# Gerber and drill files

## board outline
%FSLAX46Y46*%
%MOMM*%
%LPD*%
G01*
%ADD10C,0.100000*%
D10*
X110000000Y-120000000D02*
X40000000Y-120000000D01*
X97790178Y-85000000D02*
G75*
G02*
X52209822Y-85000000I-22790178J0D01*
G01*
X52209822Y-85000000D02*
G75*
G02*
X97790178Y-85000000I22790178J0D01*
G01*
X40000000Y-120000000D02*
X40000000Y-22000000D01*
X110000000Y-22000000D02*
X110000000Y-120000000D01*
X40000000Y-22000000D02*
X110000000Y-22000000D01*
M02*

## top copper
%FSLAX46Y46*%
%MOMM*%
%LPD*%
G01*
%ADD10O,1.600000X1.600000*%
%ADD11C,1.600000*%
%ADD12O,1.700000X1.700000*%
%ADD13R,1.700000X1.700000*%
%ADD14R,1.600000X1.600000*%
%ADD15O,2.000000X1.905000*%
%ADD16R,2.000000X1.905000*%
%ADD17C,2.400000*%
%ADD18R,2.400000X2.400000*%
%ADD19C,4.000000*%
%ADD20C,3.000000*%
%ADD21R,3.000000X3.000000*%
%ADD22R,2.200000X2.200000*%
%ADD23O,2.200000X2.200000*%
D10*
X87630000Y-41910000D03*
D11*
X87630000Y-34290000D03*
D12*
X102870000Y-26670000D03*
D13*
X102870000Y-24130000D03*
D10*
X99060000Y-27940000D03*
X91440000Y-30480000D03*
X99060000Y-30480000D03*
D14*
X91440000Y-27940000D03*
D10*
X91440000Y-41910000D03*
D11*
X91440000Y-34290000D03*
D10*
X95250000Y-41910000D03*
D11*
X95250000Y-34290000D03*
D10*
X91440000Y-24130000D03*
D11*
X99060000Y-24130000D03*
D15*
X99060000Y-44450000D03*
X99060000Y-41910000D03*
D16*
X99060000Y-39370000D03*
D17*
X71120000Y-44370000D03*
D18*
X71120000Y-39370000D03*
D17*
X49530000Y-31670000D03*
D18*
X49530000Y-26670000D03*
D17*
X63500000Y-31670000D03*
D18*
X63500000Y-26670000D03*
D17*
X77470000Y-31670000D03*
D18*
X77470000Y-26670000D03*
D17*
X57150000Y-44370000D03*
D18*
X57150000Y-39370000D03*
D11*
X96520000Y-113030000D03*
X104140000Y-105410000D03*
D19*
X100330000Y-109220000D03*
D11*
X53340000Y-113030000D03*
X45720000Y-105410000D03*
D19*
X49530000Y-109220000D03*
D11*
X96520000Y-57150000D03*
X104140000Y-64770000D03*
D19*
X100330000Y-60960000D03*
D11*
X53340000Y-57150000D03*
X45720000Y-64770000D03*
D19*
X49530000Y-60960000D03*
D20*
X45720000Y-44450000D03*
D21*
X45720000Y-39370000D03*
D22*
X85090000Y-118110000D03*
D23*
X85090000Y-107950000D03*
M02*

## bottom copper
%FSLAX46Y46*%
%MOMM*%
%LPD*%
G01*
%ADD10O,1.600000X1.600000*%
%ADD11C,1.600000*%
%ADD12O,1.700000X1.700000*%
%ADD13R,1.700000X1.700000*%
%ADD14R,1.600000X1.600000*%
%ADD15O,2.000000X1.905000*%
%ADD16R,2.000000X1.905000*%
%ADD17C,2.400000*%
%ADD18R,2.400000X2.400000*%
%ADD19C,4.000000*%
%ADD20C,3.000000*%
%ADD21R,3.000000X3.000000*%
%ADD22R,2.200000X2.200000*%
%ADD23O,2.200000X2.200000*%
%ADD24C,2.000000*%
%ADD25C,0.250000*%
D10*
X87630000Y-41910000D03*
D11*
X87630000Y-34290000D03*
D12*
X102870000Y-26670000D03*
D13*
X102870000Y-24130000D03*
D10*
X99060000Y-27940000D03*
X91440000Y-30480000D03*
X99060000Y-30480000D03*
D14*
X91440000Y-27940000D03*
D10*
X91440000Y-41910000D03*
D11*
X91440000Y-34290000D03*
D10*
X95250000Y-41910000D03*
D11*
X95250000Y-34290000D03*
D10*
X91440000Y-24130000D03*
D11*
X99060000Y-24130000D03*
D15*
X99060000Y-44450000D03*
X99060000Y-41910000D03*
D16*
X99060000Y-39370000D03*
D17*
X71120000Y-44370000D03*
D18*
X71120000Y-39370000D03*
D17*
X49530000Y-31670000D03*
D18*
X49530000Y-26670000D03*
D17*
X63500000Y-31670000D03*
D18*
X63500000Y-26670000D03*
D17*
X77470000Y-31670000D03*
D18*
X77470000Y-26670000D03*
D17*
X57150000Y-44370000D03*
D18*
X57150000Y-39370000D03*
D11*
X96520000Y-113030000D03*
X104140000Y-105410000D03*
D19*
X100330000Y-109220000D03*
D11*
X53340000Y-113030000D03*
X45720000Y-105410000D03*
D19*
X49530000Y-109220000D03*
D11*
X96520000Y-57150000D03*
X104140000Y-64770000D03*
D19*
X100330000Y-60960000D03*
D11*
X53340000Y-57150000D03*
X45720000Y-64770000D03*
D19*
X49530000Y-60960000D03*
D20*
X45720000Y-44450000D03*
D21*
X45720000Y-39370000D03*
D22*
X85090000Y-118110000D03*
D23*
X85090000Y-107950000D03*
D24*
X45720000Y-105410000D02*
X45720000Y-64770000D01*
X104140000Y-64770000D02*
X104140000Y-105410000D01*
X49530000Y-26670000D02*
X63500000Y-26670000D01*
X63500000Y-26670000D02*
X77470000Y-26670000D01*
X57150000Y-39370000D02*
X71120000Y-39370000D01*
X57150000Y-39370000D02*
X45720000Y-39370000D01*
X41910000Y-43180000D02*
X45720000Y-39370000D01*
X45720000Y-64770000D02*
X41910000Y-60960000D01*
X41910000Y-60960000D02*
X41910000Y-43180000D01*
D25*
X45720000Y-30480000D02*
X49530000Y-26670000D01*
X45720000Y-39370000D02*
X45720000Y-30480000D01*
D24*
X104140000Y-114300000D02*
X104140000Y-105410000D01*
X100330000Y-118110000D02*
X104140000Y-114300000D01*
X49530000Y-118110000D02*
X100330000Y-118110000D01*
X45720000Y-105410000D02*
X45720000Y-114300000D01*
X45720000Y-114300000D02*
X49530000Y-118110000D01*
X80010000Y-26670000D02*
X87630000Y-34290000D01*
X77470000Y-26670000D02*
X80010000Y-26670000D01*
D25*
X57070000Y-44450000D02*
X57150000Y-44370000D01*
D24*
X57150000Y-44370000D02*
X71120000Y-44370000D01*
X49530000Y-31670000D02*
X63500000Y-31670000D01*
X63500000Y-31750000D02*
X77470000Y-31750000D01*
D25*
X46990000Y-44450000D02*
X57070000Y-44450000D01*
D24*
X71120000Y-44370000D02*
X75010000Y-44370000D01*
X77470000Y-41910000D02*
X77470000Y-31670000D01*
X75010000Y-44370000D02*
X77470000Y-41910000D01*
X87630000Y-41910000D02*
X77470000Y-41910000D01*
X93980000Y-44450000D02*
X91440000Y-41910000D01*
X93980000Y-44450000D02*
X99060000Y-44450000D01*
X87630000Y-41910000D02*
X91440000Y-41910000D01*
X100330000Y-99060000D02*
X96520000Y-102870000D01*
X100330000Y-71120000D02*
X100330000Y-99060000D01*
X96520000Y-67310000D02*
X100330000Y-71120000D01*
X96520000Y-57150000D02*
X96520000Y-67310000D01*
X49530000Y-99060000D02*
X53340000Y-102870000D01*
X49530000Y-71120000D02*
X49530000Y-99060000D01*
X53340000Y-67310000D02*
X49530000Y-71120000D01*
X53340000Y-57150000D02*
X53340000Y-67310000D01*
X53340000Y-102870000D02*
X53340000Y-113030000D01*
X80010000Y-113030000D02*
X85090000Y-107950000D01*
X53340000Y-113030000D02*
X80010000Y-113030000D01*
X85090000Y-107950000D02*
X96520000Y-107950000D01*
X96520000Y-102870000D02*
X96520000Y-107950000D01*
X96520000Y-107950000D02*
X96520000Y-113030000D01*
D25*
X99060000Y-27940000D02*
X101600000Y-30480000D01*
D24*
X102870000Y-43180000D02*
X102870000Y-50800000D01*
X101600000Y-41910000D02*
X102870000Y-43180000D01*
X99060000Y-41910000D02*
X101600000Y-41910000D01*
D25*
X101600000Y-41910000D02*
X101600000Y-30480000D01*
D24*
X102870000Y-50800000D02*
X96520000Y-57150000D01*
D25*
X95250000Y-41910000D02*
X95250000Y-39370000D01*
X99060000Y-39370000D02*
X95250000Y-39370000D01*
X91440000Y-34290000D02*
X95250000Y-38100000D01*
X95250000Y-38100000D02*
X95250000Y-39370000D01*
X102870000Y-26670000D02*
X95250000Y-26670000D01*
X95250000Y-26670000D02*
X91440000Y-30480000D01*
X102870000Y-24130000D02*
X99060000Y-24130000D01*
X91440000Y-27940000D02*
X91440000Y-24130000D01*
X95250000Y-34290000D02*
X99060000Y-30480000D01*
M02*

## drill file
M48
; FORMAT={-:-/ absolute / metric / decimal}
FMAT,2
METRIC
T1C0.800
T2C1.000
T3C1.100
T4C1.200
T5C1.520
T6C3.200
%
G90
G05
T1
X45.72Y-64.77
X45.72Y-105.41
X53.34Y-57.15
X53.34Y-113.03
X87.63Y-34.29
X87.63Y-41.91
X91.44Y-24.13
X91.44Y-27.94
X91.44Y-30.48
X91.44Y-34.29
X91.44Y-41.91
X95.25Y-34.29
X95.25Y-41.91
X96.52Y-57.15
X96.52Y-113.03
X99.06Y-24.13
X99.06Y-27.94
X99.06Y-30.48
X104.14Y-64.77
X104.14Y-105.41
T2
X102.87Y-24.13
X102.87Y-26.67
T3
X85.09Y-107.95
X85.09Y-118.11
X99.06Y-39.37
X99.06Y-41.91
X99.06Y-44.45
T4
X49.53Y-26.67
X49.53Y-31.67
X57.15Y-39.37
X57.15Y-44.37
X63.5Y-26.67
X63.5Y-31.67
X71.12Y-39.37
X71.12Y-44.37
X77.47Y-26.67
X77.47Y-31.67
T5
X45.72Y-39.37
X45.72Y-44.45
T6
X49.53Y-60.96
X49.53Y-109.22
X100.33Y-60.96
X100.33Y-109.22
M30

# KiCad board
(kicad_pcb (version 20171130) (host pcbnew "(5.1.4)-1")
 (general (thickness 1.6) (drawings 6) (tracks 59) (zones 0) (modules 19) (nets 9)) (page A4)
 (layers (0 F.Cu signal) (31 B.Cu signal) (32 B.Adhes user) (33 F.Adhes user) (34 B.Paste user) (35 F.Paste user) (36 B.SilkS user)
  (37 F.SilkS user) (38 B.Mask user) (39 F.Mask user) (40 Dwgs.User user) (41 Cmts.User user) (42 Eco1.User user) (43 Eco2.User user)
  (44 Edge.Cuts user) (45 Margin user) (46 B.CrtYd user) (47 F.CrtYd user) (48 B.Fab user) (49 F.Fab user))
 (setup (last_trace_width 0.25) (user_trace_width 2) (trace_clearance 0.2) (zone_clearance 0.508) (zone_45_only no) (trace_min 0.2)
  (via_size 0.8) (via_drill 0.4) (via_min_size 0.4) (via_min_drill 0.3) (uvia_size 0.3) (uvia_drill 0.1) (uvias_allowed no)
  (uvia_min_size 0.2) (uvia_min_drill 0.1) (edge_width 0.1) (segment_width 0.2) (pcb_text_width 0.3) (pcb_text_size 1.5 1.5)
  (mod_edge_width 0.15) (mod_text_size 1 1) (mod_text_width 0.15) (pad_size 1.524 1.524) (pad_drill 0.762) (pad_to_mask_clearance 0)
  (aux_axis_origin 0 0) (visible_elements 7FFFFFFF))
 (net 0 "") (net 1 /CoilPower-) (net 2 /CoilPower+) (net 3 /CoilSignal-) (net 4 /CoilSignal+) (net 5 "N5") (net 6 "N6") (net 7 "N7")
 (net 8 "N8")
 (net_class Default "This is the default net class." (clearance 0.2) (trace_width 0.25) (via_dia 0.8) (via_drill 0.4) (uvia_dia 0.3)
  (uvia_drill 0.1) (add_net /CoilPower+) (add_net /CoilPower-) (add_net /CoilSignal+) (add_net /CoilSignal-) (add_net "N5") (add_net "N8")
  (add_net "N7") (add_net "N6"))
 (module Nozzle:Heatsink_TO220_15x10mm (layer F.Cu) (at 102.87 41.91 270)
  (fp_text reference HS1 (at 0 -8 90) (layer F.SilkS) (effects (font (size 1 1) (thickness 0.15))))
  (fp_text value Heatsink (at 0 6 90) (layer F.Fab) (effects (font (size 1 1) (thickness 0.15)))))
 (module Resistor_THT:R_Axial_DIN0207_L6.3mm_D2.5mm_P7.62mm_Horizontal (layer F.Cu) (at 87.63 34.29 270)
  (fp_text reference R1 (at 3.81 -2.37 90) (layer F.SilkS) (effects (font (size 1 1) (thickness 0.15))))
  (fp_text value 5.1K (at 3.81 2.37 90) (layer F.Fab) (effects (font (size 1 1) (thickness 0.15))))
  (pad 2 thru_hole oval (at 7.62 0 270) (size 1.6 1.6) (drill 0.8) (layers *.Cu *.Mask) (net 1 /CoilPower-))
  (pad 1 thru_hole circle (at 0 0 270) (size 1.6 1.6) (drill 0.8) (layers *.Cu *.Mask) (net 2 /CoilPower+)))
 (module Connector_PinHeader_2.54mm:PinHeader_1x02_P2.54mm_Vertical (layer F.Cu) (at 102.87 24.13)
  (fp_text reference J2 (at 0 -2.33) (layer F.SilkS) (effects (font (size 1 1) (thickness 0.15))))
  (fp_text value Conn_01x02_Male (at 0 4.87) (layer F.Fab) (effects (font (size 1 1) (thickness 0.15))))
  (pad 2 thru_hole oval (at 0 2.54) (size 1.7 1.7) (drill 1) (layers *.Cu *.Mask) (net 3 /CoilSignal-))
  (pad 1 thru_hole rect (at 0 0) (size 1.7 1.7) (drill 1) (layers *.Cu *.Mask) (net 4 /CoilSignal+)))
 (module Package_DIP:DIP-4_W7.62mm (layer F.Cu) (at 91.44 27.94)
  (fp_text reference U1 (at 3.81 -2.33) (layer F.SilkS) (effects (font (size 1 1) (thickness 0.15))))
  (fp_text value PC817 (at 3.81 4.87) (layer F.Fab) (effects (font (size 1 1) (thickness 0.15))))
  (pad 4 thru_hole oval (at 7.62 0) (size 1.6 1.6) (drill 0.8) (layers *.Cu *.Mask) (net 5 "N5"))
  (pad 2 thru_hole oval (at 0 2.54) (size 1.6 1.6) (drill 0.8) (layers *.Cu *.Mask) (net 3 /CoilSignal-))
  (pad 3 thru_hole oval (at 7.62 2.54) (size 1.6 1.6) (drill 0.8) (layers *.Cu *.Mask) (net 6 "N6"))
  (pad 1 thru_hole rect (at 0 0) (size 1.6 1.6) (drill 0.8) (layers *.Cu *.Mask) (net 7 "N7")))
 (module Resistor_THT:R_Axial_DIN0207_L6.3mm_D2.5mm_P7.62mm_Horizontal (layer F.Cu) (at 91.44 34.29 270)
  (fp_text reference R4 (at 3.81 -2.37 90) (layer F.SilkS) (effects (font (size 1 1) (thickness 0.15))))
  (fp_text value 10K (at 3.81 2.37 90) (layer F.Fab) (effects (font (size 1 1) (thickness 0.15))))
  (pad 2 thru_hole oval (at 7.62 0 270) (size 1.6 1.6) (drill 0.8) (layers *.Cu *.Mask) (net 1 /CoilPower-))
  (pad 1 thru_hole circle (at 0 0 270) (size 1.6 1.6) (drill 0.8) (layers *.Cu *.Mask) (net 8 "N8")))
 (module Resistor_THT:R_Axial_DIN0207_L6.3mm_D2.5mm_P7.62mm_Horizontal (layer F.Cu) (at 95.25 34.29 270)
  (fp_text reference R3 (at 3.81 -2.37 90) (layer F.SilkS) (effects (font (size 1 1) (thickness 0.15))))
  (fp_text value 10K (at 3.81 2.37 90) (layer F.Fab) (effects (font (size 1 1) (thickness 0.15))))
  (pad 2 thru_hole oval (at 7.62 0 270) (size 1.6 1.6) (drill 0.8) (layers *.Cu *.Mask) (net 8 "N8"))
  (pad 1 thru_hole circle (at 0 0 270) (size 1.6 1.6) (drill 0.8) (layers *.Cu *.Mask) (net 6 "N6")))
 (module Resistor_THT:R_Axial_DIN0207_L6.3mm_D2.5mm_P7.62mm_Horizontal (layer F.Cu) (at 99.06 24.13 180)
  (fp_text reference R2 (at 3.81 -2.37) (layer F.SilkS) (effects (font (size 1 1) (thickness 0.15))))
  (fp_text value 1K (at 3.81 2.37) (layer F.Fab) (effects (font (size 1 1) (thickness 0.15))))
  (pad 2 thru_hole oval (at 7.62 0 180) (size 1.6 1.6) (drill 0.8) (layers *.Cu *.Mask) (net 7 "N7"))
  (pad 1 thru_hole circle (at 0 0 180) (size 1.6 1.6) (drill 0.8) (layers *.Cu *.Mask) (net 4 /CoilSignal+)))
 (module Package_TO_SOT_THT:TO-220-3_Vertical (layer F.Cu) (at 99.06 39.37 270)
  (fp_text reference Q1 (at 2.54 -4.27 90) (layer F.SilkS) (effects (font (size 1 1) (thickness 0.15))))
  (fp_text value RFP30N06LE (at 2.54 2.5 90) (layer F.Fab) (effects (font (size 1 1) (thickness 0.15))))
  (pad 3 thru_hole oval (at 5.08 0 270) (size 1.905 2) (drill 1.1) (layers *.Cu *.Mask) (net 1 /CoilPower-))
  (pad 2 thru_hole oval (at 2.54 0 270) (size 1.905 2) (drill 1.1) (layers *.Cu *.Mask) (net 5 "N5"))
  (pad 1 thru_hole rect (at 0 0 270) (size 1.905 2) (drill 1.1) (layers *.Cu *.Mask) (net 8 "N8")))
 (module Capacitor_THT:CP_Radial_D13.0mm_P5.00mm (layer F.Cu) (at 71.12 39.37 270)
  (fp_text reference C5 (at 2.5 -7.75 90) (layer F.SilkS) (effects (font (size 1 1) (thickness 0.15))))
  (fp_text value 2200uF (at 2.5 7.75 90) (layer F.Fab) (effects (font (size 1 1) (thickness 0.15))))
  (pad 2 thru_hole circle (at 5 0 270) (size 2.4 2.4) (drill 1.2) (layers *.Cu *.Mask) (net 1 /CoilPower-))
  (pad 1 thru_hole rect (at 0 0 270) (size 2.4 2.4) (drill 1.2) (layers *.Cu *.Mask) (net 2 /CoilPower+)))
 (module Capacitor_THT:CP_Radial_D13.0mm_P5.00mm (layer F.Cu) (at 49.53 26.67 270)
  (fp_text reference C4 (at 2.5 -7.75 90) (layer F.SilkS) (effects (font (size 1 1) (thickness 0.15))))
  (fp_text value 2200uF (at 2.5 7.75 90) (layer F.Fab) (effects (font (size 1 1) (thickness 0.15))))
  (pad 2 thru_hole circle (at 5 0 270) (size 2.4 2.4) (drill 1.2) (layers *.Cu *.Mask) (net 1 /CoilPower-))
  (pad 1 thru_hole rect (at 0 0 270) (size 2.4 2.4) (drill 1.2) (layers *.Cu *.Mask) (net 2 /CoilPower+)))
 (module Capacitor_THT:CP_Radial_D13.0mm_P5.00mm (layer F.Cu) (at 63.5 26.67 270)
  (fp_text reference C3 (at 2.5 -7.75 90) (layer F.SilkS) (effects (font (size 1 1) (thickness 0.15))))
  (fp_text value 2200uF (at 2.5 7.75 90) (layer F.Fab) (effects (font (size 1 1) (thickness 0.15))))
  (pad 2 thru_hole circle (at 5 0 270) (size 2.4 2.4) (drill 1.2) (layers *.Cu *.Mask) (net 1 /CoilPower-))
  (pad 1 thru_hole rect (at 0 0 270) (size 2.4 2.4) (drill 1.2) (layers *.Cu *.Mask) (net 2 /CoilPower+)))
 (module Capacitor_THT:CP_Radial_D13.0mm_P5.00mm (layer F.Cu) (at 77.47 26.67 270)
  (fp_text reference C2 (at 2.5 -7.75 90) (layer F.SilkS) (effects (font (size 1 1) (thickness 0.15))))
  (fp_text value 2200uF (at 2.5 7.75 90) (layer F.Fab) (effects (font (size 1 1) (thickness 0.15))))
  (pad 2 thru_hole circle (at 5 0 270) (size 2.4 2.4) (drill 1.2) (layers *.Cu *.Mask) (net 1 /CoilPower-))
  (pad 1 thru_hole rect (at 0 0 270) (size 2.4 2.4) (drill 1.2) (layers *.Cu *.Mask) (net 2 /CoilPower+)))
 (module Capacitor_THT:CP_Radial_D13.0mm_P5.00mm (layer F.Cu) (at 57.15 39.37 270)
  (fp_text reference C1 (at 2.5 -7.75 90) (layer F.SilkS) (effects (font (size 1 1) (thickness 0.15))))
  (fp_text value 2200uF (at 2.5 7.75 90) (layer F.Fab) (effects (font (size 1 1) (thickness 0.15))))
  (pad 2 thru_hole circle (at 5 0 270) (size 2.4 2.4) (drill 1.2) (layers *.Cu *.Mask) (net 1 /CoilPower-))
  (pad 1 thru_hole rect (at 0 0 270) (size 2.4 2.4) (drill 1.2) (layers *.Cu *.Mask) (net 2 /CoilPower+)))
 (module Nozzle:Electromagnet (layer F.Cu) (at 100.33 109.22 180)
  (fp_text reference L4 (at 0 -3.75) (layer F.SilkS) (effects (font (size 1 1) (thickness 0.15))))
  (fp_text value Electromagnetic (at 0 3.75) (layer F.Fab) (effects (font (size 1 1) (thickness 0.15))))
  (pad 2 thru_hole circle (at 3.81 -3.81 180) (size 1.6 1.6) (drill 0.8) (layers *.Cu *.Mask) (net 5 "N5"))
  (pad 1 thru_hole circle (at -3.81 3.81 180) (size 1.6 1.6) (drill 0.8) (layers *.Cu *.Mask) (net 2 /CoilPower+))
  (pad 3 thru_hole circle (at 0 0 180) (size 4 4) (drill 3.2) (layers *.Cu *.Mask)))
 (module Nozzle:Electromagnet (layer F.Cu) (at 49.53 109.22 270)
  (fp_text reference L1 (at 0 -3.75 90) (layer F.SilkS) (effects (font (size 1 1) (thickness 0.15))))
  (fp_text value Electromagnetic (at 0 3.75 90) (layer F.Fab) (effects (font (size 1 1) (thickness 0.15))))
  (pad 2 thru_hole circle (at 3.81 -3.81 270) (size 1.6 1.6) (drill 0.8) (layers *.Cu *.Mask) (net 5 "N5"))
  (pad 1 thru_hole circle (at -3.81 3.81 270) (size 1.6 1.6) (drill 0.8) (layers *.Cu *.Mask) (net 2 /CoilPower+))
  (pad 3 thru_hole circle (at 0 0 270) (size 4 4) (drill 3.2) (layers *.Cu *.Mask)))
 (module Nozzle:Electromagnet (layer F.Cu) (at 100.33 60.96 90)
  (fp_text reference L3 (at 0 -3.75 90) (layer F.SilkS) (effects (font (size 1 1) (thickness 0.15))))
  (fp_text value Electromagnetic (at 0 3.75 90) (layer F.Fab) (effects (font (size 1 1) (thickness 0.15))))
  (pad 2 thru_hole circle (at 3.81 -3.81 90) (size 1.6 1.6) (drill 0.8) (layers *.Cu *.Mask) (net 5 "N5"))
  (pad 1 thru_hole circle (at -3.81 3.81 90) (size 1.6 1.6) (drill 0.8) (layers *.Cu *.Mask) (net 2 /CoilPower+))
  (pad 3 thru_hole circle (at 0 0 90) (size 4 4) (drill 3.2) (layers *.Cu *.Mask)))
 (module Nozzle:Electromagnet (layer F.Cu) (at 49.53 60.96)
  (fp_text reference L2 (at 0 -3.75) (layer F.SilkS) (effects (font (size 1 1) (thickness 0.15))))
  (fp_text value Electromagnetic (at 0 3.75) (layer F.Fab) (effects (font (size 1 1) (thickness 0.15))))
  (pad 2 thru_hole circle (at 3.81 -3.81) (size 1.6 1.6) (drill 0.8) (layers *.Cu *.Mask) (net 5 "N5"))
  (pad 1 thru_hole circle (at -3.81 3.81) (size 1.6 1.6) (drill 0.8) (layers *.Cu *.Mask) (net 2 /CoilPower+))
  (pad 3 thru_hole circle (at 0 0) (size 4 4) (drill 3.2) (layers *.Cu *.Mask)))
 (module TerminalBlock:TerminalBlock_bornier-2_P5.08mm (layer F.Cu) (at 45.72 39.37 270)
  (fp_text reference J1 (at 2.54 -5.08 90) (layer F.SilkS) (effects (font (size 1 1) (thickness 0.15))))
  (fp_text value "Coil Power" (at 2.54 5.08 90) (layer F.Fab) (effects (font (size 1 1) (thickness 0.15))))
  (pad 2 thru_hole circle (at 5.08 0 270) (size 3 3) (drill 1.52) (layers *.Cu *.Mask) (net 1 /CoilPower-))
  (pad 1 thru_hole rect (at 0 0 270) (size 3 3) (drill 1.52) (layers *.Cu *.Mask) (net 2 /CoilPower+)))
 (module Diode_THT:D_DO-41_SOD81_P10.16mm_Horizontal (layer F.Cu) (at 85.09 118.11 90)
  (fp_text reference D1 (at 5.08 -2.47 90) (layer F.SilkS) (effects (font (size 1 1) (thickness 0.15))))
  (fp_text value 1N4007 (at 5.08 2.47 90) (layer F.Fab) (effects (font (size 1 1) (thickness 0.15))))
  (pad 1 thru_hole rect (at 0 0 90) (size 2.2 2.2) (drill 1.1) (layers *.Cu *.Mask) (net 2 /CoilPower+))
  (pad 2 thru_hole oval (at 10.16 0 90) (size 2.2 2.2) (drill 1.1) (layers *.Cu *.Mask) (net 5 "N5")))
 (gr_line (start 110 120) (end 40 120) (layer Edge.Cuts) (width 0.1))
 (gr_circle (center 75 85) (end 97.79 85.09) (layer Edge.Cuts) (width 0.1))
 (gr_line (start 40 120) (end 40 22) (layer Edge.Cuts) (width 0.1))
 (gr_line (start 110 22) (end 110 120) (layer Edge.Cuts) (width 0.1))
 (gr_line (start 40 22) (end 110 22) (layer Edge.Cuts) (width 0.1))
 (segment (start 45.72 105.41) (end 45.72 64.77) (width 2) (layer B.Cu) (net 2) (status 30))
 (segment (start 104.14 64.77) (end 104.14 105.41) (width 2) (layer B.Cu) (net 2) (status 30))
 (segment (start 49.53 26.67) (end 63.5 26.67) (width 2) (layer B.Cu) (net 2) (status 30))
 (segment (start 63.5 26.67) (end 77.47 26.67) (width 2) (layer B.Cu) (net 2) (status 30))
 (segment (start 57.15 39.37) (end 71.12 39.37) (width 2) (layer B.Cu) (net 2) (status 30))
 (segment (start 57.15 39.37) (end 45.72 39.37) (width 2) (layer B.Cu) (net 2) (status 30))
 (segment (start 41.91 43.18) (end 45.72 39.37) (width 2) (layer B.Cu) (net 2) (status 20))
 (segment (start 45.72 64.77) (end 41.91 60.96) (width 2) (layer B.Cu) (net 2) (status 10))
 (segment (start 41.91 60.96) (end 41.91 43.18) (width 2) (layer B.Cu) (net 2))
 (segment (start 45.72 30.48) (end 49.53 26.67) (width 0.25) (layer B.Cu) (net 2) (status 20))
 (segment (start 45.72 39.37) (end 45.72 30.48) (width 0.25) (layer B.Cu) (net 2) (status 10))
 (segment (start 104.14 114.3) (end 104.14 105.41) (width 2) (layer B.Cu) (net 2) (status 20))
 (segment (start 100.33 118.11) (end 104.14 114.3) (width 2) (layer B.Cu) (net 2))
 (segment (start 49.53 118.11) (end 100.33 118.11) (width 2) (layer B.Cu) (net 2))
 (segment (start 45.72 105.41) (end 45.72 114.3) (width 2) (layer B.Cu) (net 2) (status 10))
 (segment (start 45.72 114.3) (end 49.53 118.11) (width 2) (layer B.Cu) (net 2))
 (segment (start 80.01 26.67) (end 87.63 34.29) (width 2) (layer B.Cu) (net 2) (status 20))
 (segment (start 77.47 26.67) (end 80.01 26.67) (width 2) (layer B.Cu) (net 2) (status 10))
 (segment (start 57.07 44.45) (end 57.15 44.37) (width 0.25) (layer B.Cu) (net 1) (status 30))
 (segment (start 57.15 44.37) (end 71.12 44.37) (width 2) (layer B.Cu) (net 1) (status 30))
 (segment (start 49.53 31.67) (end 63.5 31.67) (width 2) (layer B.Cu) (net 1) (status 30))
 (segment (start 63.5 31.75) (end 77.47 31.75) (width 2) (layer B.Cu) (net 1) (status 30))
 (segment (start 46.99 44.45) (end 57.07 44.45) (width 0.25) (layer B.Cu) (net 1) (status 30))
 (segment (start 71.12 44.37) (end 75.01 44.37) (width 2) (layer B.Cu) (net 1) (status 10))
 (segment (start 77.47 41.91) (end 77.47 31.67) (width 2) (layer B.Cu) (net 1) (status 20))
 (segment (start 75.01 44.37) (end 77.47 41.91) (width 2) (layer B.Cu) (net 1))
 (segment (start 87.63 41.91) (end 77.47 41.91) (width 2) (layer B.Cu) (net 1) (status 10))
 (segment (start 93.98 44.45) (end 91.44 41.91) (width 2) (layer B.Cu) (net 1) (status 20))
 (segment (start 93.98 44.45) (end 99.06 44.45) (width 2) (layer B.Cu) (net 1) (status 20))
 (segment (start 87.63 41.91) (end 91.44 41.91) (width 2) (layer B.Cu) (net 1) (status 30))
 (segment (start 100.33 99.06) (end 96.52 102.87) (width 2) (layer B.Cu) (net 5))
 (segment (start 100.33 71.12) (end 100.33 99.06) (width 2) (layer B.Cu) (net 5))
 (segment (start 96.52 67.31) (end 100.33 71.12) (width 2) (layer B.Cu) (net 5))
 (segment (start 96.52 57.15) (end 96.52 67.31) (width 2) (layer B.Cu) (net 5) (status 10))
 (segment (start 49.53 99.06) (end 53.34 102.87) (width 2) (layer B.Cu) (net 5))
 (segment (start 49.53 71.12) (end 49.53 99.06) (width 2) (layer B.Cu) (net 5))
 (segment (start 53.34 67.31) (end 49.53 71.12) (width 2) (layer B.Cu) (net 5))
 (segment (start 53.34 57.15) (end 53.34 67.31) (width 2) (layer B.Cu) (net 5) (status 10))
 (segment (start 53.34 102.87) (end 53.34 113.03) (width 2) (layer B.Cu) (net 5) (status 20))
 (segment (start 80.01 113.03) (end 85.09 107.95) (width 2) (layer B.Cu) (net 5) (status 20))
 (segment (start 53.34 113.03) (end 80.01 113.03) (width 2) (layer B.Cu) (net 5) (status 10))
 (segment (start 85.09 107.95) (end 96.52 107.95) (width 2) (layer B.Cu) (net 5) (status 10))
 (segment (start 96.52 102.87) (end 96.52 107.95) (width 2) (layer B.Cu) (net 5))
 (segment (start 96.52 107.95) (end 96.52 113.03) (width 2) (layer B.Cu) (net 5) (status 20))
 (segment (start 99.06 27.94) (end 101.6 30.48) (width 0.25) (layer B.Cu) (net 5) (status 10))
 (segment (start 102.87 43.18) (end 102.87 50.8) (width 2) (layer B.Cu) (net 5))
 (segment (start 101.6 41.91) (end 102.87 43.18) (width 2) (layer B.Cu) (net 5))
 (segment (start 99.06 41.91) (end 101.6 41.91) (width 2) (layer B.Cu) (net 5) (status 10))
 (segment (start 101.6 41.91) (end 101.6 30.48) (width 0.25) (layer B.Cu) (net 5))
 (segment (start 102.87 50.8) (end 96.52 57.15) (width 2) (layer B.Cu) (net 5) (status 20))
 (segment (start 95.25 41.91) (end 95.25 39.37) (width 0.25) (layer B.Cu) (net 8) (status 10))
 (segment (start 99.06 39.37) (end 95.25 39.37) (width 0.25) (layer B.Cu) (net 8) (status 10))
 (segment (start 91.44 34.29) (end 95.25 38.1) (width 0.25) (layer B.Cu) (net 8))
 (segment (start 95.25 38.1) (end 95.25 39.37) (width 0.25) (layer B.Cu) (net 8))
 (segment (start 102.87 26.67) (end 95.25 26.67) (width 0.25) (layer B.Cu) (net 3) (status 10))
 (segment (start 95.25 26.67) (end 91.44 30.48) (width 0.25) (layer B.Cu) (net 3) (status 20))
 (segment (start 102.87 24.13) (end 99.06 24.13) (width 0.25) (layer B.Cu) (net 4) (status 30))
 (segment (start 91.44 27.94) (end 91.44 24.13) (width 0.25) (layer B.Cu) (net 7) (status 30))
 (segment (start 95.25 34.29) (end 99.06 30.48) (width 0.25) (layer B.Cu) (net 6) (status 30)))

